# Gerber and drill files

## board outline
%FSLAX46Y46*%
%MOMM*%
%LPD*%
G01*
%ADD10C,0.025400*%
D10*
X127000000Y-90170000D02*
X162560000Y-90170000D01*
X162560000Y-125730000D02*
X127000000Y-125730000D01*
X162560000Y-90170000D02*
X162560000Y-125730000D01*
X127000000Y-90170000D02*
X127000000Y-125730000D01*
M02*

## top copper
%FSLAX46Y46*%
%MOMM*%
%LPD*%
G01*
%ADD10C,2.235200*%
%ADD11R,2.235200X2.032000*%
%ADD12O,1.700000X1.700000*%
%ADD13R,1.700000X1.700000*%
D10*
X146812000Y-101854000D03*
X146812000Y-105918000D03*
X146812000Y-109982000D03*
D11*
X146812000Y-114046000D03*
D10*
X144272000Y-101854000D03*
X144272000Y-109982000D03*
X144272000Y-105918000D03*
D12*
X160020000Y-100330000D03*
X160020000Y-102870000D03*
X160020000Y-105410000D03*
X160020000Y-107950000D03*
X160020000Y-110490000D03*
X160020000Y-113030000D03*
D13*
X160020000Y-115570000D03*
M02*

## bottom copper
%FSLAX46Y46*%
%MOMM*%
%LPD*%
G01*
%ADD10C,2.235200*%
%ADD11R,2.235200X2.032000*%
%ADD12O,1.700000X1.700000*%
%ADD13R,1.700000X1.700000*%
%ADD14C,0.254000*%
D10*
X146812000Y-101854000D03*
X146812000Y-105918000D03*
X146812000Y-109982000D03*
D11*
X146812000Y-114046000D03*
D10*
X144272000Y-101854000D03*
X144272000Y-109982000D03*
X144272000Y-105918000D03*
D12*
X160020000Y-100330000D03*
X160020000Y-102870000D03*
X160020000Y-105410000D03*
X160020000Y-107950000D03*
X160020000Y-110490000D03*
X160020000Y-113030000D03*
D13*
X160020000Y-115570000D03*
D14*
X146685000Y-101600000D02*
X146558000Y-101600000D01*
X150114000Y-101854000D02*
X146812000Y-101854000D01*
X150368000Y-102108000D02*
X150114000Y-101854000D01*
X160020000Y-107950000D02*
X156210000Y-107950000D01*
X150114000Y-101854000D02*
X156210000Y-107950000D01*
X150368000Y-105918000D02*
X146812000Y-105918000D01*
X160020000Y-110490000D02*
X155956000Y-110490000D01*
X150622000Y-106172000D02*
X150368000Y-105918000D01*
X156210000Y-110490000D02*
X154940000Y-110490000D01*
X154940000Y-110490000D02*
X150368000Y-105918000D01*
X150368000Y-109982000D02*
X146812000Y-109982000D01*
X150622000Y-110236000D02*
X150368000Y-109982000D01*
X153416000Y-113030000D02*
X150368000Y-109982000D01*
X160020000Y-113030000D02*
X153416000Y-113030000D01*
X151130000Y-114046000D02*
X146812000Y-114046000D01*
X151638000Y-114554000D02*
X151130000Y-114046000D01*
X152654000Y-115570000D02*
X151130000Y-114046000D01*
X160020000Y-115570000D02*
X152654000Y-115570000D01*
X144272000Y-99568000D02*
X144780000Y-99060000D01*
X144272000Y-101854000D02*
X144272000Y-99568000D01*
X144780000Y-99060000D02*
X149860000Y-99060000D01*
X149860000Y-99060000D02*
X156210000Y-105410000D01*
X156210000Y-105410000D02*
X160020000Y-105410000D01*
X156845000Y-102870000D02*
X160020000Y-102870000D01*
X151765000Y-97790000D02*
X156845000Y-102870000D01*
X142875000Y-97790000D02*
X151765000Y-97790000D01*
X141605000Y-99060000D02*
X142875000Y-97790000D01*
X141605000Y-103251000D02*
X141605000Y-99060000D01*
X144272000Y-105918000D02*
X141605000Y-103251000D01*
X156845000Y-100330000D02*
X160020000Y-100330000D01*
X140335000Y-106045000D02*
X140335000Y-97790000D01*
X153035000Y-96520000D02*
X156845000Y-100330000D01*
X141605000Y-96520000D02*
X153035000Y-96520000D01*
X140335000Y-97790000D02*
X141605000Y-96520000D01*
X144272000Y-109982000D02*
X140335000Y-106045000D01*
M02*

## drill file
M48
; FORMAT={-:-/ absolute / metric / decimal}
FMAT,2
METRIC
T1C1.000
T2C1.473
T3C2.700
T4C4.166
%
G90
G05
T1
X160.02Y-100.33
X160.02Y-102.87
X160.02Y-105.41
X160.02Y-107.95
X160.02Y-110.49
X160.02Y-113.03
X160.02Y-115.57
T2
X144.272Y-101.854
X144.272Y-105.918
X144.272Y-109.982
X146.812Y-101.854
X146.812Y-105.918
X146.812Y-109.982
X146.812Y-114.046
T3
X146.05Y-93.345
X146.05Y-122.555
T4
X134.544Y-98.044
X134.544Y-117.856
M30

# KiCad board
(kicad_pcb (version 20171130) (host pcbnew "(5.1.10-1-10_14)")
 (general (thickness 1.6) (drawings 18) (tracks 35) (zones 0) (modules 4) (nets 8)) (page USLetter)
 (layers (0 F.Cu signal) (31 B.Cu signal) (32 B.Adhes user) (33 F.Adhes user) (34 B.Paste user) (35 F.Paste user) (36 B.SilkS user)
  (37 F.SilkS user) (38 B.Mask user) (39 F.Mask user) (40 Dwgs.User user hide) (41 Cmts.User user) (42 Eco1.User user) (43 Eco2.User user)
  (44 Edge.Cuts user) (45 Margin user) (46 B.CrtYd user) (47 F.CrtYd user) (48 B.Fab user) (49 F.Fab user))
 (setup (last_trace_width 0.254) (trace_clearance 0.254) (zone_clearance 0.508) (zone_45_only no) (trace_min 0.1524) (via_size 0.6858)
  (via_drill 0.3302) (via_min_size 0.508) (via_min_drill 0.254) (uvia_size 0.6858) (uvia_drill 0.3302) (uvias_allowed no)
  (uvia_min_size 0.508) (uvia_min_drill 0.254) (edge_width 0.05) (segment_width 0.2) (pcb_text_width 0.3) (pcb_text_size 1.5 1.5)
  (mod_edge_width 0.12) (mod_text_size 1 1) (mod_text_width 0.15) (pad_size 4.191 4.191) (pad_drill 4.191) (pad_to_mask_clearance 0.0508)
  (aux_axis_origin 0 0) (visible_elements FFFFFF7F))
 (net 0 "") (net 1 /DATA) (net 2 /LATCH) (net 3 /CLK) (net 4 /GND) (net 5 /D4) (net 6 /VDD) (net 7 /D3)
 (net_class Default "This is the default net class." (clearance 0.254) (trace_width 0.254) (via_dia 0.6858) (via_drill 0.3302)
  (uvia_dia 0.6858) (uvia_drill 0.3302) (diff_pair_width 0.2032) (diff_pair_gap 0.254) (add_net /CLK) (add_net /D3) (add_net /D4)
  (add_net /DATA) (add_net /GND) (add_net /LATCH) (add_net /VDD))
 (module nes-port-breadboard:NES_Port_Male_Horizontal (layer F.Cu) (at 147.574 107.95)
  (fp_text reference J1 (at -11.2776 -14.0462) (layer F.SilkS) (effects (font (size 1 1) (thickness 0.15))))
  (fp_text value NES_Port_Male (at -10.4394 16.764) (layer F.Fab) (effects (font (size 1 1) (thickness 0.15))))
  (pad 4 thru_hole circle (at -0.762 -6.096) (size 2.2352 2.2352) (drill 1.4732) (layers *.Cu *.Mask) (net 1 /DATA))
  (pad 3 thru_hole circle (at -0.762 -2.032) (size 2.2352 2.2352) (drill 1.4732) (layers *.Cu *.Mask) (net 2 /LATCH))
  (pad 2 thru_hole circle (at -0.762 2.032) (size 2.2352 2.2352) (drill 1.4732) (layers *.Cu *.Mask) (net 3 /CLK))
  (pad 1 thru_hole rect (at -0.762 6.096) (size 2.2352 2.032) (drill 1.4732) (layers *.Cu *.Mask) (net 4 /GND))
  (pad 5 thru_hole circle (at -3.302 -6.096) (size 2.2352 2.2352) (drill 1.4732) (layers *.Cu *.Mask) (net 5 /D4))
  (pad 7 thru_hole circle (at -3.302 2.032) (size 2.2352 2.2352) (drill 1.4732) (layers *.Cu *.Mask) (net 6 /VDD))
  (pad 6 thru_hole circle (at -3.302 -2.032) (size 2.2352 2.2352) (drill 1.4732) (layers *.Cu *.Mask) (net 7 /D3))
  (pad "" np_thru_hole circle (at -13.0302 -9.906) (size 4.1656 4.1656) (drill 4.1656) (layers *.Cu *.Mask))
  (pad "" np_thru_hole circle (at -13.0302 9.906) (size 4.1656 4.1656) (drill 4.1656) (layers *.Cu *.Mask)))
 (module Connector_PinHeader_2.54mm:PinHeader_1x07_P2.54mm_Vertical (layer B.Cu) (at 160.02 115.57)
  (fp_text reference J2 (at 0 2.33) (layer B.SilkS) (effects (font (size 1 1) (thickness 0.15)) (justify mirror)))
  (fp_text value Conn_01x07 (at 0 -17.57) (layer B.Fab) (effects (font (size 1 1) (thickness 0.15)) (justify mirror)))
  (pad 7 thru_hole oval (at 0 -15.24) (size 1.7 1.7) (drill 1) (layers *.Cu *.Mask) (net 6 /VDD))
  (pad 6 thru_hole oval (at 0 -12.7) (size 1.7 1.7) (drill 1) (layers *.Cu *.Mask) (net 7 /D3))
  (pad 5 thru_hole oval (at 0 -10.16) (size 1.7 1.7) (drill 1) (layers *.Cu *.Mask) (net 5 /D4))
  (pad 4 thru_hole oval (at 0 -7.62) (size 1.7 1.7) (drill 1) (layers *.Cu *.Mask) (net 1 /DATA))
  (pad 3 thru_hole oval (at 0 -5.08) (size 1.7 1.7) (drill 1) (layers *.Cu *.Mask) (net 2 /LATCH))
  (pad 2 thru_hole oval (at 0 -2.54) (size 1.7 1.7) (drill 1) (layers *.Cu *.Mask) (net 3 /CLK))
  (pad 1 thru_hole rect (at 0 0) (size 1.7 1.7) (drill 1) (layers *.Cu *.Mask) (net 4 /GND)))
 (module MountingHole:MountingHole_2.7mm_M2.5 (layer F.Cu) (at 146.05 122.555)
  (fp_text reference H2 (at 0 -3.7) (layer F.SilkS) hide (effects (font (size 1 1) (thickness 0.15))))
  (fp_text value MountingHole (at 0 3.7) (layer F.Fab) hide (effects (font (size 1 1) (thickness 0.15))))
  (pad 1 np_thru_hole circle (at 0 0) (size 2.7 2.7) (drill 2.7) (layers *.Cu *.Mask)))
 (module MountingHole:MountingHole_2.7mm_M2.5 (layer F.Cu) (at 146.05 93.345)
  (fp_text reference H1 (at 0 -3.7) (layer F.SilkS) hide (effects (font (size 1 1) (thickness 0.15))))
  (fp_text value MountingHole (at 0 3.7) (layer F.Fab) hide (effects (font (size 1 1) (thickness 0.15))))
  (pad 1 np_thru_hole circle (at 0 0) (size 2.7 2.7) (drill 2.7) (layers *.Cu *.Mask)))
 (gr_line (start 127 90.17) (end 162.56 90.17) (layer Edge.Cuts) (width 0.0254))
 (gr_line (start 162.56 125.73) (end 127 125.73) (layer Edge.Cuts) (width 0.0254))
 (gr_line (start 162.56 90.17) (end 162.56 125.73) (layer Edge.Cuts) (width 0.0254))
 (gr_line (start 127 90.17) (end 127 125.73) (layer Edge.Cuts) (width 0.0254))
 (segment (start 146.685 101.6) (end 146.558 101.6) (width 0.254) (layer B.Cu) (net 1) (status 30))
 (segment (start 150.114 101.854) (end 146.812 101.854) (width 0.254) (layer B.Cu) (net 1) (status 20))
 (segment (start 150.368 102.108) (end 150.114 101.854) (width 0.254) (layer B.Cu) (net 1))
 (segment (start 160.02 107.95) (end 156.21 107.95) (width 0.254) (layer B.Cu) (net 1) (status 10))
 (segment (start 150.114 101.854) (end 156.21 107.95) (width 0.254) (layer B.Cu) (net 1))
 (segment (start 150.368 105.918) (end 146.812 105.918) (width 0.254) (layer B.Cu) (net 2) (status 20))
 (segment (start 160.02 110.49) (end 155.956 110.49) (width 0.254) (layer B.Cu) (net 2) (status 10))
 (segment (start 150.622 106.172) (end 150.368 105.918) (width 0.254) (layer B.Cu) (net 2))
 (segment (start 156.21 110.49) (end 154.94 110.49) (width 0.254) (layer B.Cu) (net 2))
 (segment (start 154.94 110.49) (end 150.368 105.918) (width 0.254) (layer B.Cu) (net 2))
 (segment (start 150.368 109.982) (end 146.812 109.982) (width 0.254) (layer B.Cu) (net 3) (status 20))
 (segment (start 150.622 110.236) (end 150.368 109.982) (width 0.254) (layer B.Cu) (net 3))
 (segment (start 153.416 113.03) (end 150.368 109.982) (width 0.254) (layer B.Cu) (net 3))
 (segment (start 160.02 113.03) (end 153.416 113.03) (width 0.254) (layer B.Cu) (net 3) (status 10))
 (segment (start 151.13 114.046) (end 146.812 114.046) (width 0.254) (layer B.Cu) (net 4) (status 20))
 (segment (start 151.638 114.554) (end 151.13 114.046) (width 0.254) (layer B.Cu) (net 4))
 (segment (start 152.654 115.57) (end 151.13 114.046) (width 0.254) (layer B.Cu) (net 4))
 (segment (start 160.02 115.57) (end 152.654 115.57) (width 0.254) (layer B.Cu) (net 4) (status 10))
 (segment (start 144.272 99.568) (end 144.78 99.06) (width 0.254) (layer B.Cu) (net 5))
 (segment (start 144.272 101.854) (end 144.272 99.568) (width 0.254) (layer B.Cu) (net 5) (status 10))
 (segment (start 144.78 99.06) (end 149.86 99.06) (width 0.254) (layer B.Cu) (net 5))
 (segment (start 149.86 99.06) (end 156.21 105.41) (width 0.254) (layer B.Cu) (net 5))
 (segment (start 156.21 105.41) (end 160.02 105.41) (width 0.254) (layer B.Cu) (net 5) (status 20))
 (segment (start 156.845 102.87) (end 160.02 102.87) (width 0.254) (layer B.Cu) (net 7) (status 20))
 (segment (start 151.765 97.79) (end 156.845 102.87) (width 0.254) (layer B.Cu) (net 7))
 (segment (start 142.875 97.79) (end 151.765 97.79) (width 0.254) (layer B.Cu) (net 7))
 (segment (start 141.605 99.06) (end 142.875 97.79) (width 0.254) (layer B.Cu) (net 7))
 (segment (start 141.605 103.251) (end 141.605 99.06) (width 0.254) (layer B.Cu) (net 7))
 (segment (start 144.272 105.918) (end 141.605 103.251) (width 0.254) (layer B.Cu) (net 7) (status 10))
 (segment (start 156.845 100.33) (end 160.02 100.33) (width 0.254) (layer B.Cu) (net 6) (status 20))
 (segment (start 140.335 106.045) (end 140.335 97.79) (width 0.254) (layer B.Cu) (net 6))
 (segment (start 153.035 96.52) (end 156.845 100.33) (width 0.254) (layer B.Cu) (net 6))
 (segment (start 141.605 96.52) (end 153.035 96.52) (width 0.254) (layer B.Cu) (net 6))
 (segment (start 140.335 97.79) (end 141.605 96.52) (width 0.254) (layer B.Cu) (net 6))
 (segment (start 144.272 109.982) (end 140.335 106.045) (width 0.254) (layer B.Cu) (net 6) (status 10)))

